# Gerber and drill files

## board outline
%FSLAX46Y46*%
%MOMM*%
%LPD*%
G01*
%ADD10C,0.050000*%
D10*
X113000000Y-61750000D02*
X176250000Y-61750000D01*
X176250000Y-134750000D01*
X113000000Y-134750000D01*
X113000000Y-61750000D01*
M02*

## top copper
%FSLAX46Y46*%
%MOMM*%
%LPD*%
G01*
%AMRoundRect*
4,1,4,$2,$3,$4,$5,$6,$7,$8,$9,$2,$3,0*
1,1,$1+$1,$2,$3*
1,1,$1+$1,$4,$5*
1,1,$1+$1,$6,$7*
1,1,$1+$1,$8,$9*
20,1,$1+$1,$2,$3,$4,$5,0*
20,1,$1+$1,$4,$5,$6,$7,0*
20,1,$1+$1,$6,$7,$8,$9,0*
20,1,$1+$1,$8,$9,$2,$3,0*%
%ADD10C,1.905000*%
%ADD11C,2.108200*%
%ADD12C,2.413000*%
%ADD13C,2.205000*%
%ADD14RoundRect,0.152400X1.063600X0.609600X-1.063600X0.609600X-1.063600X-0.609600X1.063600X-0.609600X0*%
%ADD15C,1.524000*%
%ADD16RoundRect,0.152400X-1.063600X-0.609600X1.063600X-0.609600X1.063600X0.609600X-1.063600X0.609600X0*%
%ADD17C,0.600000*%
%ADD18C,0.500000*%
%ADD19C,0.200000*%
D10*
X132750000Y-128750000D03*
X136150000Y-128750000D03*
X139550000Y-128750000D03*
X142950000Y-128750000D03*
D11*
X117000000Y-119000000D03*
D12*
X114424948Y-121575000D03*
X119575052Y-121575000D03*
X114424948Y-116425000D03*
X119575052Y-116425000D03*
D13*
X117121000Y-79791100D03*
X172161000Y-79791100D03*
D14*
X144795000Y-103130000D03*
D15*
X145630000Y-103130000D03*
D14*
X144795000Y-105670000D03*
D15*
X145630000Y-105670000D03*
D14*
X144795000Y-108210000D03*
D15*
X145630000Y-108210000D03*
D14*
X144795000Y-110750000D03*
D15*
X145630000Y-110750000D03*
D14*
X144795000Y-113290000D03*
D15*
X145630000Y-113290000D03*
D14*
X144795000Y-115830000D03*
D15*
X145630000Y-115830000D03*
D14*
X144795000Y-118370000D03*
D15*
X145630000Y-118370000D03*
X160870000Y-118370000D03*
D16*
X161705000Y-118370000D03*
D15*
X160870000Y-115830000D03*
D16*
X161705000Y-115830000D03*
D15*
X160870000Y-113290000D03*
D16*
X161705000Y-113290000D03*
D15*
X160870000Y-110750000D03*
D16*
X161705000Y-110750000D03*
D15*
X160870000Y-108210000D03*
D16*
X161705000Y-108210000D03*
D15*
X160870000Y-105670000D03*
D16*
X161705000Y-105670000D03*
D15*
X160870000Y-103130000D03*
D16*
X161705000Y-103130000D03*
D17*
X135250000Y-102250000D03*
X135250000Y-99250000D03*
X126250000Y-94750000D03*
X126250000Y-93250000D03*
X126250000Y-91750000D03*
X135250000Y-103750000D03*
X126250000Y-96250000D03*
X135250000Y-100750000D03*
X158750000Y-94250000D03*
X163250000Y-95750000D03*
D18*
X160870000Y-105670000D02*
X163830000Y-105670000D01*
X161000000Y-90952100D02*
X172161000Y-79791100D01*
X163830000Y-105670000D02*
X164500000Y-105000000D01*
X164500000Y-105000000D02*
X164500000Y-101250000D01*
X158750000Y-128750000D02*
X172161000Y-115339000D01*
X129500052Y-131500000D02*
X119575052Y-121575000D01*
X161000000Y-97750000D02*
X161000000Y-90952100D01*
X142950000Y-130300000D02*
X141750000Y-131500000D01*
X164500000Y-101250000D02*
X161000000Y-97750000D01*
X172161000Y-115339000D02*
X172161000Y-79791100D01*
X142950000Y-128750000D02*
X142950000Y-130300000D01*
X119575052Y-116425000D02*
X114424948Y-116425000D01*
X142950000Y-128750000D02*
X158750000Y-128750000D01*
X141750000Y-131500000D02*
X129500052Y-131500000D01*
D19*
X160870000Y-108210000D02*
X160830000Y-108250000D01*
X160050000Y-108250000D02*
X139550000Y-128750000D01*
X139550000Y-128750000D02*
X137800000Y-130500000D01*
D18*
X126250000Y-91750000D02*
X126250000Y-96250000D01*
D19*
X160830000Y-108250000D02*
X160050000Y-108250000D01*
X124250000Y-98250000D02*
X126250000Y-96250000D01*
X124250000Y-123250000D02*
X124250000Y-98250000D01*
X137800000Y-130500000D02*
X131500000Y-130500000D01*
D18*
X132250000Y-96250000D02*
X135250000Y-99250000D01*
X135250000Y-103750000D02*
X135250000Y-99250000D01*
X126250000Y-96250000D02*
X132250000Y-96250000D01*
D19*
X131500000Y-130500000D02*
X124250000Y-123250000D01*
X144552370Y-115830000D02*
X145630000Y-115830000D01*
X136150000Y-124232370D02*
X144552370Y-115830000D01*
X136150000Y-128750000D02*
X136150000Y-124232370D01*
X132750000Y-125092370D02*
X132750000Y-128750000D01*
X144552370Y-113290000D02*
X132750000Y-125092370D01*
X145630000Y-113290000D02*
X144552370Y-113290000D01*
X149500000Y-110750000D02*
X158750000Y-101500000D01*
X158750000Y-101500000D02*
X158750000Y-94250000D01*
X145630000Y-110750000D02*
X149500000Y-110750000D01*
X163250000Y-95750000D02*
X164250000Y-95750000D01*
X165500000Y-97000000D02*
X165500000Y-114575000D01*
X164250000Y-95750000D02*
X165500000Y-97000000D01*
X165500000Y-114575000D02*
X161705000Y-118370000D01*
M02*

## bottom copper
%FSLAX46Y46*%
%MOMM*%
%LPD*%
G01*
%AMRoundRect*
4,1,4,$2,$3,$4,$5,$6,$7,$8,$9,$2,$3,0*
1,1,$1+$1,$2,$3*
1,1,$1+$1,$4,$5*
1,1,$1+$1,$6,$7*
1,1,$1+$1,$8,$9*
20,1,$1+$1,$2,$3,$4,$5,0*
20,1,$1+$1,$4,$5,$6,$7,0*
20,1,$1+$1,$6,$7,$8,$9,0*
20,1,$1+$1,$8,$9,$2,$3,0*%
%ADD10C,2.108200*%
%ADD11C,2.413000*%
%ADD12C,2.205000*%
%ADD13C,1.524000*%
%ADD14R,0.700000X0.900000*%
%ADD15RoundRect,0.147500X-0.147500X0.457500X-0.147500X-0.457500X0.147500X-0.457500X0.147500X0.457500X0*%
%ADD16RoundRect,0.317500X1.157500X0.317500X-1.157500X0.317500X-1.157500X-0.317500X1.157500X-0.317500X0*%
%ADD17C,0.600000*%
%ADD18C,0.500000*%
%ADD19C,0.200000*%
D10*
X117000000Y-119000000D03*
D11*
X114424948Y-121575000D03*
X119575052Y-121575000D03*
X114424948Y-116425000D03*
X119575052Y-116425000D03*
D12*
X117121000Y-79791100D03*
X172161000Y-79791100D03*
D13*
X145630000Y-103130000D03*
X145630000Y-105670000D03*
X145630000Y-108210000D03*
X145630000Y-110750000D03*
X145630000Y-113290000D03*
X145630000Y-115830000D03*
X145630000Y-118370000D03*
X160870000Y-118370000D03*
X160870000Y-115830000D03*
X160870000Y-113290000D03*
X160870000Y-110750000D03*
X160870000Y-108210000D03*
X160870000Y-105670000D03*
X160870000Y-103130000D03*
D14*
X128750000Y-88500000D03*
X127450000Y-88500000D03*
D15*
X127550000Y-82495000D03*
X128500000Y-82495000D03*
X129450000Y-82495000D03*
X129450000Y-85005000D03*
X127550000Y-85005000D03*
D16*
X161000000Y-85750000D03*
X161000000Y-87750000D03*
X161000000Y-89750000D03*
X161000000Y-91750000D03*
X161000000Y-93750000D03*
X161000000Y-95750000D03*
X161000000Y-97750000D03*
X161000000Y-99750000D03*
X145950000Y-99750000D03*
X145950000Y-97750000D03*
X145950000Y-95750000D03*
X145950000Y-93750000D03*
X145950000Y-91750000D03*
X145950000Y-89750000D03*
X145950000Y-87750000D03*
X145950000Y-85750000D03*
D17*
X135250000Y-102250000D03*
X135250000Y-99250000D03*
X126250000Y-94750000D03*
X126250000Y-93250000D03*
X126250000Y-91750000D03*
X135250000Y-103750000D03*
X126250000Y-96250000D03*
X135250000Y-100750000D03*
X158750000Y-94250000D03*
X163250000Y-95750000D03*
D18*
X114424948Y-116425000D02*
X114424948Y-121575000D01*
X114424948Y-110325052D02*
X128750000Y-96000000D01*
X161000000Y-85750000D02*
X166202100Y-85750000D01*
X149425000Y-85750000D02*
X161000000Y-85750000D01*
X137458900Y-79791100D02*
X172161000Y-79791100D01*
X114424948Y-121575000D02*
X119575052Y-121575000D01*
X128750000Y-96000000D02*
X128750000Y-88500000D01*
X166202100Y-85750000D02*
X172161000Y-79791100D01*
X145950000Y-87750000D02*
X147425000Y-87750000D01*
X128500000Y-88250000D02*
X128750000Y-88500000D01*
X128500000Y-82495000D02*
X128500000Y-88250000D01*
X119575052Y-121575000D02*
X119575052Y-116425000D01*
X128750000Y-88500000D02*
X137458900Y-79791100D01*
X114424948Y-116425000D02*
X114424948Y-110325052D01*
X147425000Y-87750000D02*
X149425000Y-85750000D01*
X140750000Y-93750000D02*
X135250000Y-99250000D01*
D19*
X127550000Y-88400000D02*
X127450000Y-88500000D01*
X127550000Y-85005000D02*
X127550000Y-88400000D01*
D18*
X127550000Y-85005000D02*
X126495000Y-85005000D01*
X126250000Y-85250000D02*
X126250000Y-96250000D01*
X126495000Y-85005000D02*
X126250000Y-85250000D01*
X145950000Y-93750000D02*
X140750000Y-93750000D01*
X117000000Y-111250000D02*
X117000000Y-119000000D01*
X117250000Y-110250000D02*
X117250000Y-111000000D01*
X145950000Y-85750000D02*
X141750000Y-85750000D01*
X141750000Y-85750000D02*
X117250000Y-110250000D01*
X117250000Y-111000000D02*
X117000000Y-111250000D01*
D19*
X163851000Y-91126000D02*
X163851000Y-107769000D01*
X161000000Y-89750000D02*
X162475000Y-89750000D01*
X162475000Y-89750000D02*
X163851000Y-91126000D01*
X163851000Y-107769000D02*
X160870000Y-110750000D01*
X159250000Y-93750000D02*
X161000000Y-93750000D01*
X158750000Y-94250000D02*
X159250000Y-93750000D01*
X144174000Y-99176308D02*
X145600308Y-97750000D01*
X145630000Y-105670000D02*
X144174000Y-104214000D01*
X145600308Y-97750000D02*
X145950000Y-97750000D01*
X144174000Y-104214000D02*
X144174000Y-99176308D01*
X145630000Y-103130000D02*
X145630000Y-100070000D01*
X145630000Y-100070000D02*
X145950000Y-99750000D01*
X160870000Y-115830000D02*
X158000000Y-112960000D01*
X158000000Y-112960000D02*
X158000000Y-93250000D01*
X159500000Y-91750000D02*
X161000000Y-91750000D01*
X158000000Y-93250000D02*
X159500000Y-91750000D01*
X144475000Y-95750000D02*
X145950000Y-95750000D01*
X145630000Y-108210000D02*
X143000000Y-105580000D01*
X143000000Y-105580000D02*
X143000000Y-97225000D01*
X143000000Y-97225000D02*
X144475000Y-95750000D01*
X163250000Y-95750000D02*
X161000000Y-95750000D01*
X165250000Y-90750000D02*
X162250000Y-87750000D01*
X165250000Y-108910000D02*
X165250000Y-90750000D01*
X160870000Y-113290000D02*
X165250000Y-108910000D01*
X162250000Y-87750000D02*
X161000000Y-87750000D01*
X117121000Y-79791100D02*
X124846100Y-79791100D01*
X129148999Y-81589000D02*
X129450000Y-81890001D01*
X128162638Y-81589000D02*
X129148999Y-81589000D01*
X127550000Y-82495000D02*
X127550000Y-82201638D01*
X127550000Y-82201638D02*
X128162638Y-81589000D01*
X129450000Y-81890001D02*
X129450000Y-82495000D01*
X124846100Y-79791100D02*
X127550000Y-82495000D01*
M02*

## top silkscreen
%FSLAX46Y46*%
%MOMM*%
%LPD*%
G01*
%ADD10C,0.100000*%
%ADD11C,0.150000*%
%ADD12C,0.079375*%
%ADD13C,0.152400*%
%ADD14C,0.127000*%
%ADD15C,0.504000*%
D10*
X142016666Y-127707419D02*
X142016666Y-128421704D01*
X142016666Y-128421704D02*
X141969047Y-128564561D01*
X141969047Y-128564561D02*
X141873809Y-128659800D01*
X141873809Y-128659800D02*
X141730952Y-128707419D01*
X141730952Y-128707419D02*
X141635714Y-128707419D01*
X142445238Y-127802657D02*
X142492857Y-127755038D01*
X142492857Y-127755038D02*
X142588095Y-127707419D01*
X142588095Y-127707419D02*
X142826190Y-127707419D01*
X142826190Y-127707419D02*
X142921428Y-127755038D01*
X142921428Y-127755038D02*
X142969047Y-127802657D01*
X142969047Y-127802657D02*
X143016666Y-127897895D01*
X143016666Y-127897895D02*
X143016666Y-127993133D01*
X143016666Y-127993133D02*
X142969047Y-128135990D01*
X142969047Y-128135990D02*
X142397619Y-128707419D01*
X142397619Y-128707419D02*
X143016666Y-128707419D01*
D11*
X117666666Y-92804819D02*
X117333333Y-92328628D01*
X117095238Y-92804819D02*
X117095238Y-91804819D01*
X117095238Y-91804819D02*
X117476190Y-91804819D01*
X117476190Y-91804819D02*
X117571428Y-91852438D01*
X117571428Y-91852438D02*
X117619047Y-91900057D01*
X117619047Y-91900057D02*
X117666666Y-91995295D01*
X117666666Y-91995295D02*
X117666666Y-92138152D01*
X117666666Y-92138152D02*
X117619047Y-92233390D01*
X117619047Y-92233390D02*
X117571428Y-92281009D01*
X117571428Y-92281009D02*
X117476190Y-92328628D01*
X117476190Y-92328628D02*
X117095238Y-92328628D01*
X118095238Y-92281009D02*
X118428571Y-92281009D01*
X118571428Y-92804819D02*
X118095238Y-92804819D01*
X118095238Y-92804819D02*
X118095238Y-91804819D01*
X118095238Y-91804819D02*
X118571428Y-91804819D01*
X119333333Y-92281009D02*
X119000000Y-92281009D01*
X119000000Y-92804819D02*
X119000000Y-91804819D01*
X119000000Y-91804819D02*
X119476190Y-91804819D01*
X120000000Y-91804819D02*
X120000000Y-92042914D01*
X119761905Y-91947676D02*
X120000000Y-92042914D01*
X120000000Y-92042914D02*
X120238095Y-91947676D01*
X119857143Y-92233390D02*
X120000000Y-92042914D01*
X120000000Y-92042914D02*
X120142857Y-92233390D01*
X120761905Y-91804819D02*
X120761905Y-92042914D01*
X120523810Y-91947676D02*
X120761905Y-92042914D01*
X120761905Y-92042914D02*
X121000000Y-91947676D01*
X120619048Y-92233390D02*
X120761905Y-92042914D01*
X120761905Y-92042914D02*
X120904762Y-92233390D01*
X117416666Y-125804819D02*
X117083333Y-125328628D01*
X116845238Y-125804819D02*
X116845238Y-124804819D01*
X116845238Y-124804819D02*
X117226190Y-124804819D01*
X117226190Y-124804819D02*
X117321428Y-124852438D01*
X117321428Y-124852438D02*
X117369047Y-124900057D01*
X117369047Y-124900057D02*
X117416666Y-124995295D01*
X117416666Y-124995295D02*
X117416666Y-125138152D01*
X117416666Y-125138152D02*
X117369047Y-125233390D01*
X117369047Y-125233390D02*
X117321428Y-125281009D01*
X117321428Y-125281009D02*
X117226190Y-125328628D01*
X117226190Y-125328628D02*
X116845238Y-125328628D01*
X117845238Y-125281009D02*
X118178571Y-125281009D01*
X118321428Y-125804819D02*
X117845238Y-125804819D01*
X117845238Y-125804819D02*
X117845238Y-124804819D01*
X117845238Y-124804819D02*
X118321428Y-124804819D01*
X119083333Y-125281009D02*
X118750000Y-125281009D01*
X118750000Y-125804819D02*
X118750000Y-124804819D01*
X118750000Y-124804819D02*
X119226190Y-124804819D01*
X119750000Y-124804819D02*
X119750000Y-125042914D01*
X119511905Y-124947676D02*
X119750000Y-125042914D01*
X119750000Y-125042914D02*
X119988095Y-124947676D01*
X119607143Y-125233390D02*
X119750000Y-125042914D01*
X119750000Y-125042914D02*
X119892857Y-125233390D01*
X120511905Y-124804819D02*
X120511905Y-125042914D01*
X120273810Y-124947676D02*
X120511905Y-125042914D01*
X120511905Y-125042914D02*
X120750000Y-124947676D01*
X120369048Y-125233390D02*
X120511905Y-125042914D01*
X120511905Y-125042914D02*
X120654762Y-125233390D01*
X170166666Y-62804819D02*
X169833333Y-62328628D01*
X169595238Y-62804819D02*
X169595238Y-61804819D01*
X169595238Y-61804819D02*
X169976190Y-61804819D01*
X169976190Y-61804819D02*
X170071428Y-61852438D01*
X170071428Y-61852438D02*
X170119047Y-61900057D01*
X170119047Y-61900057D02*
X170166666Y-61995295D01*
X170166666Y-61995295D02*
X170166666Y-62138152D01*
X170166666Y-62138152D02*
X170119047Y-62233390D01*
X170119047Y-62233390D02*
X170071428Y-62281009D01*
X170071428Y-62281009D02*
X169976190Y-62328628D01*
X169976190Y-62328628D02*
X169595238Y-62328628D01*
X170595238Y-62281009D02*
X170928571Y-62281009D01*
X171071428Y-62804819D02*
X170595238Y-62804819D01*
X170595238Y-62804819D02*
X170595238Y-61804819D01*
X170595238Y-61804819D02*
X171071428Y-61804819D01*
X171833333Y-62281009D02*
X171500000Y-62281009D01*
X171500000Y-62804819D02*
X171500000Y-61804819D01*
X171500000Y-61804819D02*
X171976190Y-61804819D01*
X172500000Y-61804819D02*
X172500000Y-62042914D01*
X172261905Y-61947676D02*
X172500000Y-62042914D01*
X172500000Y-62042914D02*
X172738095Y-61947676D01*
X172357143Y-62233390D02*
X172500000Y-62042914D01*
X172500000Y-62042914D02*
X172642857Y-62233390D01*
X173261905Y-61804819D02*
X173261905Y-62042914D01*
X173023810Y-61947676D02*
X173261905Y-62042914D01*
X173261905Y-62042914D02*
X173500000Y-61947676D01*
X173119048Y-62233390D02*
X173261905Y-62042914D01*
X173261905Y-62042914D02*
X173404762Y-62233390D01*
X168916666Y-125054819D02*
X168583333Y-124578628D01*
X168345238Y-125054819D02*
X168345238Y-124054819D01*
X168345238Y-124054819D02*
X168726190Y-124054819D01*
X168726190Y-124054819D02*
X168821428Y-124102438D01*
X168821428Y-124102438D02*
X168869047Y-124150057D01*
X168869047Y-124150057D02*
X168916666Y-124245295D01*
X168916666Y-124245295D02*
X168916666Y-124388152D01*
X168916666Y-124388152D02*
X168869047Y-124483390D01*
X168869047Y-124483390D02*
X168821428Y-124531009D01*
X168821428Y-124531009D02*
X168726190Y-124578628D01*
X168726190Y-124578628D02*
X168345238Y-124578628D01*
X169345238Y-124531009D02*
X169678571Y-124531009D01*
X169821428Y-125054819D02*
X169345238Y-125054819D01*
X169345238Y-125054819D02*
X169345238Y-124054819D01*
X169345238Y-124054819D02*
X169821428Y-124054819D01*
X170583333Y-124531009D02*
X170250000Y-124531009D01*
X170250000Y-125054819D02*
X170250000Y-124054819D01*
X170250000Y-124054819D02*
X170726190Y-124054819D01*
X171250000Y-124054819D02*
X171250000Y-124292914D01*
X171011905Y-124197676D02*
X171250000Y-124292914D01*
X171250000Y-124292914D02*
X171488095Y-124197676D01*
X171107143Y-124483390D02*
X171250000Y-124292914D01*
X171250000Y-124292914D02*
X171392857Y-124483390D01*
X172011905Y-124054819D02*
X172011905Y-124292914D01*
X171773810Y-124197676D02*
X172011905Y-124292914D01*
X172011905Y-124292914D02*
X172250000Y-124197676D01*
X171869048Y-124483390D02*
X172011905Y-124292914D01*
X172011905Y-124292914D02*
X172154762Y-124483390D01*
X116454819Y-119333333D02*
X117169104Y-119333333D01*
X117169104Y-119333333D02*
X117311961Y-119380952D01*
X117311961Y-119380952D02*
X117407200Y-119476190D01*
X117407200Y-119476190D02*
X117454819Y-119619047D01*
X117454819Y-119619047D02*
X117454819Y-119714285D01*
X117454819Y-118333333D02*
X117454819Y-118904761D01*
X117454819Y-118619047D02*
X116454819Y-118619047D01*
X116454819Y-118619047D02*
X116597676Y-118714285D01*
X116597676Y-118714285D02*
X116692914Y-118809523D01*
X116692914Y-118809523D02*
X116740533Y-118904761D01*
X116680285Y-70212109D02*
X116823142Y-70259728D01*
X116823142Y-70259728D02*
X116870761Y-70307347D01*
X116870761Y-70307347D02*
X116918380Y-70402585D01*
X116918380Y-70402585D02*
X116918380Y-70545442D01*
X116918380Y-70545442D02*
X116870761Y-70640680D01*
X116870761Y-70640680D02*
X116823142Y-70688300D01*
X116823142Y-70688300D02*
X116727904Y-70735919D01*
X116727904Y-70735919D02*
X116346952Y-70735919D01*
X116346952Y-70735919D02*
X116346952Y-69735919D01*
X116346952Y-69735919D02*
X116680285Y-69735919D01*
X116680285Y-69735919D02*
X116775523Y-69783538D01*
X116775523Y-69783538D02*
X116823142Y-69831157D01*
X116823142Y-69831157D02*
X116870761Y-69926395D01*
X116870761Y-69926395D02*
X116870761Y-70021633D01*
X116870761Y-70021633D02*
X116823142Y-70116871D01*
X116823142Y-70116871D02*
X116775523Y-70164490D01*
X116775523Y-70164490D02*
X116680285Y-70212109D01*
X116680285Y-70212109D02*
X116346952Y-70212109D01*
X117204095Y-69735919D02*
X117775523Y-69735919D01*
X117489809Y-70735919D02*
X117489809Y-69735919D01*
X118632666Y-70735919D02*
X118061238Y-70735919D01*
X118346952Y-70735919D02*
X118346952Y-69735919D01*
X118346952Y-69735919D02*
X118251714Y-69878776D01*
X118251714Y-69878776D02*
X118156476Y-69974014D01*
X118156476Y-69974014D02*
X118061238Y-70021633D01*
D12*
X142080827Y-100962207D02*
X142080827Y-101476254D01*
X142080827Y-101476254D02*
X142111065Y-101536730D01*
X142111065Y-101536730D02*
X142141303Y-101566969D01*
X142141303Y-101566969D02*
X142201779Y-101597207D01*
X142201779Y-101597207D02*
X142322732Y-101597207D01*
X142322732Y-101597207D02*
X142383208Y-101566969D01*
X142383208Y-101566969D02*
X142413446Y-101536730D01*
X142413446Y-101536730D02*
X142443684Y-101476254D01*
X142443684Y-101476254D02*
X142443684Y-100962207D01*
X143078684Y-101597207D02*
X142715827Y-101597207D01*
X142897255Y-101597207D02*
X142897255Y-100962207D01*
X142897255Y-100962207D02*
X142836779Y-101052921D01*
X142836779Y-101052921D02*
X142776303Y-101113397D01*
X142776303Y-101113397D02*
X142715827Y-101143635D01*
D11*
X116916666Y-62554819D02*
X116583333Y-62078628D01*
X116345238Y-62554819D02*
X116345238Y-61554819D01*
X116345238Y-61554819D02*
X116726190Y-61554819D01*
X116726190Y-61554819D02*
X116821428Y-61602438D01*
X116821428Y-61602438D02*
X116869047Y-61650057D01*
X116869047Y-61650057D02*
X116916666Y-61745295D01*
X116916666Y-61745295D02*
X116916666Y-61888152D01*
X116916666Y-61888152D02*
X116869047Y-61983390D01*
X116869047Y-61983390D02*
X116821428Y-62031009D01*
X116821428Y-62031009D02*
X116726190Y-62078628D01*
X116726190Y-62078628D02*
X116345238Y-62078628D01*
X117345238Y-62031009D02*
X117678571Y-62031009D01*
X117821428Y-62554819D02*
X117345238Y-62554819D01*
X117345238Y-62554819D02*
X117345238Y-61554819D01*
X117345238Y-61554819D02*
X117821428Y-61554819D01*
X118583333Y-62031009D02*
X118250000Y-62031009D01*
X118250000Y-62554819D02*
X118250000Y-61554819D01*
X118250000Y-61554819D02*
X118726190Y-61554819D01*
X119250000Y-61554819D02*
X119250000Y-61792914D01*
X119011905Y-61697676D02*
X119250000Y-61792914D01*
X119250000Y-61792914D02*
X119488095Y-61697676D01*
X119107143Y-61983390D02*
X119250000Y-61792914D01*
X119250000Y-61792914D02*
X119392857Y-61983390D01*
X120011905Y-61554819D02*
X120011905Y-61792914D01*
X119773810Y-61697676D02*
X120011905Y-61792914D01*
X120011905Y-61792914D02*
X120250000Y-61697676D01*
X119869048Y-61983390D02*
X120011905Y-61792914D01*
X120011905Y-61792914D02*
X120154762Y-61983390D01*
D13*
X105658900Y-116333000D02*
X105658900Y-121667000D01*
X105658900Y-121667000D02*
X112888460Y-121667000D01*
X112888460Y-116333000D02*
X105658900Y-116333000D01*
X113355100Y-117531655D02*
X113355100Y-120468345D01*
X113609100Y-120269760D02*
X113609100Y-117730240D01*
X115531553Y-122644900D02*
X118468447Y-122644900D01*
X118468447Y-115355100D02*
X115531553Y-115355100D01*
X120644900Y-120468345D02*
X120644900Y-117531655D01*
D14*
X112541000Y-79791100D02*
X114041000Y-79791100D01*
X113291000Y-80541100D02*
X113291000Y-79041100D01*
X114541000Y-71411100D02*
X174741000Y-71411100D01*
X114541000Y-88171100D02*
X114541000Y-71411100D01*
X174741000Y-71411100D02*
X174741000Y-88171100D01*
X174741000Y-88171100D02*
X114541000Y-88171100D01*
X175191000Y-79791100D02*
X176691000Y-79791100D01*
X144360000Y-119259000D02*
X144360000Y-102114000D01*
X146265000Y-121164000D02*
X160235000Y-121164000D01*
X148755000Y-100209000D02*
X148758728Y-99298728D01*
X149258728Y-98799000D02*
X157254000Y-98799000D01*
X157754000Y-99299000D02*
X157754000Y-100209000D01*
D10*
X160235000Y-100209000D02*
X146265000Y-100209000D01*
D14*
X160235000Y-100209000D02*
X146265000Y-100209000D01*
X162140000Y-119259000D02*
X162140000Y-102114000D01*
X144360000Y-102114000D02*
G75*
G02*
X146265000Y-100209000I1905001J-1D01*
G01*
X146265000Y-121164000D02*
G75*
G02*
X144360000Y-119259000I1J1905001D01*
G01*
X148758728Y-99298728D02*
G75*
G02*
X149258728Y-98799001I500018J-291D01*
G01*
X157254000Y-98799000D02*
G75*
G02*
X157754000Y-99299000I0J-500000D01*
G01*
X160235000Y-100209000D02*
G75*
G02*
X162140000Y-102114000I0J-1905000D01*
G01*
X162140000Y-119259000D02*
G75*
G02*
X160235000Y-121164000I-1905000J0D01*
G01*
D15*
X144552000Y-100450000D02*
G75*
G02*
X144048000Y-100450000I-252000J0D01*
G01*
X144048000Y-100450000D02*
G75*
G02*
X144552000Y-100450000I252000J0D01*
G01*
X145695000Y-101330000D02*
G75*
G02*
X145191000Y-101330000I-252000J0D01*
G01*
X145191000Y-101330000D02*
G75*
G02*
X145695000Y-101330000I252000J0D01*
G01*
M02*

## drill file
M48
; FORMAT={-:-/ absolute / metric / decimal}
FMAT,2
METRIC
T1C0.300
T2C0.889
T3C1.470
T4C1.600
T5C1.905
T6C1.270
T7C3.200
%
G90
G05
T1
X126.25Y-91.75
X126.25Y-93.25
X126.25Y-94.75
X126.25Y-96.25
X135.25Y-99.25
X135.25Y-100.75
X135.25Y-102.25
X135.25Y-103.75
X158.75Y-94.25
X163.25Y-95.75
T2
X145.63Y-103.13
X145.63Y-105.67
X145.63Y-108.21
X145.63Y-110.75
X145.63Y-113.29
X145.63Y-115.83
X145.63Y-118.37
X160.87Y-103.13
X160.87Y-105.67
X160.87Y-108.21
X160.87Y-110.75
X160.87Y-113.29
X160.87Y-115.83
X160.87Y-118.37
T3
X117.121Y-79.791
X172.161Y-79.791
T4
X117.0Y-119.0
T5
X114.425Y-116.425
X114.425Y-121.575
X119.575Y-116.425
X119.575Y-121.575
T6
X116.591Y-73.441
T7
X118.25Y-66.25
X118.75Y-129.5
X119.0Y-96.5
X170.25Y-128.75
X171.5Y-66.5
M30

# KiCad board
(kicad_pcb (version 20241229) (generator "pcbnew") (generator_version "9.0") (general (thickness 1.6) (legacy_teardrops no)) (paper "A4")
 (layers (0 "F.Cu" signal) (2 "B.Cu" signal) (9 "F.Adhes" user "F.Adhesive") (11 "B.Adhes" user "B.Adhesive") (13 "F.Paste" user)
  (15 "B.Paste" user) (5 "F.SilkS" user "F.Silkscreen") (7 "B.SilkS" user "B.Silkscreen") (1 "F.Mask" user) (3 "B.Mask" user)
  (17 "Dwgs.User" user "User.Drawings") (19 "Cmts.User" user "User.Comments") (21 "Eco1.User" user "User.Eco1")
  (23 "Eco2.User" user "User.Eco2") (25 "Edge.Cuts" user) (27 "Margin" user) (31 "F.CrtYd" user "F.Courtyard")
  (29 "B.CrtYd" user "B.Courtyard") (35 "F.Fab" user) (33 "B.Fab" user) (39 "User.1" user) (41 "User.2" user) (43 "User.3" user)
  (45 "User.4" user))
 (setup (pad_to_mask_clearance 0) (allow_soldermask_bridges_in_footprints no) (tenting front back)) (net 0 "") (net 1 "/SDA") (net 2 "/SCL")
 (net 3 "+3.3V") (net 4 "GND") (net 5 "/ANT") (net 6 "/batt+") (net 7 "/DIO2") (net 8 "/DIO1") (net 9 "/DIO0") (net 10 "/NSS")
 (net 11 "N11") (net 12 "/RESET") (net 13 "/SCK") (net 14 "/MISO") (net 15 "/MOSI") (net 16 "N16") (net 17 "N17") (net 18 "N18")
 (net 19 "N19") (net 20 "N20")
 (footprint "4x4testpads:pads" (layer "F.Cu") (at 142.35 128.75)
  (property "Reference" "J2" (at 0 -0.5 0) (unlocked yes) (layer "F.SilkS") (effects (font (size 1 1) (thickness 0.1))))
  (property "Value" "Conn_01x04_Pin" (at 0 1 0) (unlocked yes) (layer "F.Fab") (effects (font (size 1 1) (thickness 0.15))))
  (pad "1" smd circle (at -9.6 0) (size 1.905 1.905) (layers "F.Cu" "F.Mask" "F.Paste") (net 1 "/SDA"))
  (pad "2" smd circle (at -6.2 0) (size 1.905 1.905) (layers "F.Cu" "F.Mask" "F.Paste") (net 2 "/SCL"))
  (pad "3" smd circle (at -2.8 0) (size 1.905 1.905) (layers "F.Cu" "F.Mask" "F.Paste") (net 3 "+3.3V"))
  (pad "4" smd circle (at 0.6 0) (size 1.905 1.905) (layers "F.Cu" "F.Mask" "F.Paste") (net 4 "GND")))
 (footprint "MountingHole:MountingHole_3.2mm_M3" (layer "F.Cu") (at 119 96.5)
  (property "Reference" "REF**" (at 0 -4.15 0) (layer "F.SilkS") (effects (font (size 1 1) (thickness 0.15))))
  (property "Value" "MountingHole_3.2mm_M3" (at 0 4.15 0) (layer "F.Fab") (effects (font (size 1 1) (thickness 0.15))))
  (pad "" np_thru_hole circle (at 0 0) (size 3.2 3.2) (drill 3.2) (layers "*.Cu" "*.Mask")))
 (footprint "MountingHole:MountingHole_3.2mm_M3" (layer "F.Cu") (at 118.75 129.5)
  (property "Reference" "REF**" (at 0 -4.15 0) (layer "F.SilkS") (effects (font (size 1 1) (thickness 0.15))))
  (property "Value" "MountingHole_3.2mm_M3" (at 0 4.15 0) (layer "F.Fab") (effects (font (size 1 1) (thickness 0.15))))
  (pad "" np_thru_hole circle (at 0 0) (size 3.2 3.2) (drill 3.2) (layers "*.Cu" "*.Mask")))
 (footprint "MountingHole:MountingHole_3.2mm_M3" (layer "F.Cu") (at 171.5 66.5)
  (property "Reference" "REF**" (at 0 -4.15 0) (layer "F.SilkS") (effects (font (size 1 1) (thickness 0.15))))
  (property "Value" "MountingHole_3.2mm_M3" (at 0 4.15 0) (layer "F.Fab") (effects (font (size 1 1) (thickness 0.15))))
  (pad "" np_thru_hole circle (at 0 0) (size 3.2 3.2) (drill 3.2) (layers "*.Cu" "*.Mask")))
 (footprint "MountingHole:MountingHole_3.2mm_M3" (layer "F.Cu") (at 170.25 128.75)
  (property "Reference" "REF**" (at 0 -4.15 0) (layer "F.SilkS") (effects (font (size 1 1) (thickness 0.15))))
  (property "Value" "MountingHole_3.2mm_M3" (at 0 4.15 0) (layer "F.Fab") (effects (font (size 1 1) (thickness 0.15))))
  (pad "" np_thru_hole circle (at 0 0) (size 3.2 3.2) (drill 3.2) (layers "*.Cu" "*.Mask")))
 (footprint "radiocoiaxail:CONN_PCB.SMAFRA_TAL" (layer "F.Cu") (at 117 119 90)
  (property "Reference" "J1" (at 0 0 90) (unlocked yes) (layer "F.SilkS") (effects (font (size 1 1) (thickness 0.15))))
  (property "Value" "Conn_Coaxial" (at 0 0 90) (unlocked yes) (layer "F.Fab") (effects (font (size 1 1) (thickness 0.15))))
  (fp_line (start 2.667 -11.3411) (end -2.667 -11.3411) (stroke (width 0.1524) (type solid)) (layer "F.SilkS"))
  (fp_line (start -2.667 -11.3411) (end -2.667 -4.11154) (stroke (width 0.1524) (type solid)) (layer "F.SilkS"))
  (fp_line (start 2.667 -4.11154) (end 2.667 -11.3411) (stroke (width 0.1524) (type solid)) (layer "F.SilkS"))
  (fp_line (start 1.468345 -3.6449) (end -1.468345 -3.6449) (stroke (width 0.1524) (type solid)) (layer "F.SilkS"))
  (fp_line (start -1.26976 -3.3909) (end 1.26976 -3.3909) (stroke (width 0.1524) (type solid)) (layer "F.SilkS"))
  (fp_line (start -3.6449 -1.468447) (end -3.6449 1.468447) (stroke (width 0.1524) (type solid)) (layer "F.SilkS"))
  (fp_line (start 3.6449 1.468447) (end 3.6449 -1.468447) (stroke (width 0.1524) (type solid)) (layer "F.SilkS"))
  (fp_line (start -1.468345 3.6449) (end 1.468345 3.6449) (stroke (width 0.1524) (type solid)) (layer "F.SilkS"))
  (pad "1" thru_hole circle (at 0 0 90) (size 2.1082 2.1082) (drill 1.6002) (layers "*.Cu" "*.Mask") (remove_unused_layers no)
   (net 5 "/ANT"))
  (pad "2" thru_hole circle (at -2.575 -2.575052 90) (size 2.413 2.413) (drill 1.905) (layers "*.Cu" "*.Mask") (remove_unused_layers no)
   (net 4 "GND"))
  (pad "2" thru_hole circle (at -2.575 2.575052 90) (size 2.413 2.413) (drill 1.905) (layers "*.Cu" "*.Mask") (remove_unused_layers no)
   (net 4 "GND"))
  (pad "2" thru_hole circle (at 2.575 -2.575052 90) (size 2.413 2.413) (drill 1.905) (layers "*.Cu" "*.Mask") (remove_unused_layers no)
   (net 4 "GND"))
  (pad "2" thru_hole circle (at 2.575 2.575052 90) (size 2.413 2.413) (drill 1.905) (layers "*.Cu" "*.Mask") (remove_unused_layers no)
   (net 4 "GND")))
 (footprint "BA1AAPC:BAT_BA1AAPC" (layer "F.Cu") (at 144.641 79.7911)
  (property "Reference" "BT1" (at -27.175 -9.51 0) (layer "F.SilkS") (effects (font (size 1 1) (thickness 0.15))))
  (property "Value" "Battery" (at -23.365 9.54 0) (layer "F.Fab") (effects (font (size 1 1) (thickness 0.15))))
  (fp_line (start -32.1 0) (end -30.6 0) (stroke (width 0.127) (type solid)) (layer "F.SilkS"))
  (fp_line (start -31.35 0.75) (end -31.35 -0.75) (stroke (width 0.127) (type solid)) (layer "F.SilkS"))
  (fp_line (start -30.1 -8.38) (end 30.1 -8.38) (stroke (width 0.127) (type solid)) (layer "F.SilkS"))
  (fp_line (start -30.1 8.38) (end -30.1 -8.38) (stroke (width 0.127) (type solid)) (layer "F.SilkS"))
  (fp_line (start 30.1 -8.38) (end 30.1 8.38) (stroke (width 0.127) (type solid)) (layer "F.SilkS"))
  (fp_line (start 30.1 8.38) (end -30.1 8.38) (stroke (width 0.127) (type solid)) (layer "F.SilkS"))
  (fp_line (start 30.55 0) (end 32.05 0) (stroke (width 0.127) (type solid)) (layer "F.SilkS"))
  (pad "" np_thru_hole circle (at -28.05 -6.35) (size 1.27 1.27) (drill 1.27) (layers "*.Cu" "*.Mask"))
  (pad "1" thru_hole circle (at -27.52 0) (size 2.205 2.205) (drill 1.47) (layers "*.Cu" "*.Mask") (remove_unused_layers no)
   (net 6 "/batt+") (solder_mask_margin 0.102))
  (pad "2" thru_hole circle (at 27.52 0) (size 2.205 2.205) (drill 1.47) (layers "*.Cu" "*.Mask") (remove_unused_layers no) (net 4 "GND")
   (solder_mask_margin 0.102)))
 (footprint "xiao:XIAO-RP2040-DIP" (layer "F.Cu") (at 153.25 110.75)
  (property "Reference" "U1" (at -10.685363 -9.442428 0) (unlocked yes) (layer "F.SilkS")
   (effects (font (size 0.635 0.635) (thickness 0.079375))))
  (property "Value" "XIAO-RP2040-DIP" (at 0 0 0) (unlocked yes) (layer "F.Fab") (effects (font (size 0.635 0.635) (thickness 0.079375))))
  (fp_line (start -8.89 8.509) (end -8.89 -8.636) (stroke (width 0.127) (type solid)) (layer "F.SilkS"))
  (fp_line (start -6.985 10.414) (end 6.985 10.414) (stroke (width 0.127) (type solid)) (layer "F.SilkS"))
  (fp_line (start -4.495 -10.541) (end -4.491272 -11.451272) (stroke (width 0.127) (type solid)) (layer "F.SilkS"))
  (fp_line (start -3.991272 -11.951) (end 4.004 -11.951) (stroke (width 0.127) (type solid)) (layer "F.SilkS"))
  (fp_line (start 4.504 -11.451) (end 4.504 -10.541) (stroke (width 0.127) (type solid)) (layer "F.SilkS"))
  (fp_line (start 6.985 -10.541) (end -6.985 -10.541) (stroke (width 0.1) (type solid)) (layer "F.SilkS"))
  (fp_line (start 6.985 -10.541) (end -6.985 -10.541) (stroke (width 0.127) (type solid)) (layer "F.SilkS"))
  (fp_line (start 8.89 8.509) (end 8.89 -8.636) (stroke (width 0.127) (type solid)) (layer "F.SilkS"))
  (fp_arc (start -8.89 -8.636) (mid -8.332038 -9.983038) (end -6.985 -10.541) (stroke (width 0.127) (type solid)) (layer "F.SilkS"))
  (fp_arc (start -6.985 10.414) (mid -8.332038 9.856038) (end -8.89 8.509) (stroke (width 0.127) (type solid)) (layer "F.SilkS"))
  (fp_arc (start -4.491272 -11.451272) (mid -4.344728 -11.80464) (end -3.991272 -11.951) (stroke (width 0.127) (type default))
   (layer "F.SilkS"))
  (fp_arc (start 4.004 -11.951) (mid 4.357553 -11.804553) (end 4.504 -11.451) (stroke (width 0.127) (type default)) (layer "F.SilkS"))
  (fp_arc (start 6.985 -10.541) (mid 8.332038 -9.983038) (end 8.89 -8.636) (stroke (width 0.127) (type solid)) (layer "F.SilkS"))
  (fp_arc (start 8.89 8.509) (mid 8.332038 9.856038) (end 6.985 10.414) (stroke (width 0.127) (type solid)) (layer "F.SilkS"))
  (fp_circle (center -8.95 -10.3) (end -8.95 -10.554) (stroke (width 0.5) (type solid)) (fill yes) (layer "F.SilkS"))
  (fp_circle (center -7.807 -9.42) (end -7.807 -9.674) (stroke (width 0.5) (type solid)) (fill yes) (layer "F.SilkS"))
  (pad "1" smd roundrect (at -8.455 -7.62 180) (size 2.432 1.524) (layers "F.Cu" "F.Mask") (roundrect_rratio 0.1) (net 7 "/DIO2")
   (thermal_bridge_angle 45))
  (pad "1" thru_hole circle (at -7.62 -7.62 180) (size 1.524 1.524) (drill 0.889) (layers "*.Cu" "*.Mask") (remove_unused_layers no)
   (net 7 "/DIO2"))
  (pad "2" smd roundrect (at -8.455 -5.08 180) (size 2.432 1.524) (layers "F.Cu" "F.Mask") (roundrect_rratio 0.1) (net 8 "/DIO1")
   (thermal_bridge_angle 45))
  (pad "2" thru_hole circle (at -7.62 -5.08 180) (size 1.524 1.524) (drill 0.889) (layers "*.Cu" "*.Mask") (remove_unused_layers no)
   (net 8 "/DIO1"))
  (pad "3" smd roundrect (at -8.455 -2.54 180) (size 2.432 1.524) (layers "F.Cu" "F.Mask") (roundrect_rratio 0.1) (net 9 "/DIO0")
   (thermal_bridge_angle 45))
  (pad "3" thru_hole circle (at -7.62 -2.54 180) (size 1.524 1.524) (drill 0.889) (layers "*.Cu" "*.Mask") (remove_unused_layers no)
   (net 9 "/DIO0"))
  (pad "4" smd roundrect (at -8.455 0 180) (size 2.432 1.524) (layers "F.Cu" "F.Mask") (roundrect_rratio 0.1) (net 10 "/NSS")
   (thermal_bridge_angle 45))
  (pad "4" thru_hole circle (at -7.62 0 180) (size 1.524 1.524) (drill 0.889) (layers "*.Cu" "*.Mask") (remove_unused_layers no)
   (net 10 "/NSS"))
  (pad "5" smd roundrect (at -8.455 2.54 180) (size 2.432 1.524) (layers "F.Cu" "F.Mask") (roundrect_rratio 0.1) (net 1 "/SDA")
   (thermal_bridge_angle 45))
  (pad "5" thru_hole circle (at -7.62 2.54 180) (size 1.524 1.524) (drill 0.889) (layers "*.Cu" "*.Mask") (remove_unused_layers no)
   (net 1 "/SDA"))
  (pad "6" smd roundrect (at -8.455 5.08 180) (size 2.432 1.524) (layers "F.Cu" "F.Mask") (roundrect_rratio 0.1) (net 2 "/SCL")
   (thermal_bridge_angle 45))
  (pad "6" thru_hole circle (at -7.62 5.08 180) (size 1.524 1.524) (drill 0.889) (layers "*.Cu" "*.Mask") (remove_unused_layers no)
   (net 2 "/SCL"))
  (pad "7" smd roundrect (at -8.455 7.62 180) (size 2.432 1.524) (layers "F.Cu" "F.Mask") (roundrect_rratio 0.1) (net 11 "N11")
   (thermal_bridge_angle 45))
  (pad "7" thru_hole circle (at -7.62 7.62 180) (size 1.524 1.524) (drill 0.889) (layers "*.Cu" "*.Mask") (remove_unused_layers no)
   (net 11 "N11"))
  (pad "8" thru_hole circle (at 7.62 7.62) (size 1.524 1.524) (drill 0.889) (layers "*.Cu" "*.Mask") (remove_unused_layers no)
   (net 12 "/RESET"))
  (pad "8" smd roundrect (at 8.455 7.62) (size 2.432 1.524) (layers "F.Cu" "F.Mask") (roundrect_rratio 0.1) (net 12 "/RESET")
   (thermal_bridge_angle 45))
  (pad "9" thru_hole circle (at 7.62 5.08) (size 1.524 1.524) (drill 0.889) (layers "*.Cu" "*.Mask") (remove_unused_layers no)
   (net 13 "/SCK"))
  (pad "9" smd roundrect (at 8.455 5.08) (size 2.432 1.524) (layers "F.Cu" "F.Mask") (roundrect_rratio 0.1) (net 13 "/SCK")
   (thermal_bridge_angle 45))
  (pad "10" thru_hole circle (at 7.62 2.54) (size 1.524 1.524) (drill 0.889) (layers "*.Cu" "*.Mask") (remove_unused_layers no)
   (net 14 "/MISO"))
  (pad "10" smd roundrect (at 8.455 2.54) (size 2.432 1.524) (layers "F.Cu" "F.Mask") (roundrect_rratio 0.1) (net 14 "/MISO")
   (thermal_bridge_angle 45))
  (pad "11" thru_hole circle (at 7.62 0) (size 1.524 1.524) (drill 0.889) (layers "*.Cu" "*.Mask") (remove_unused_layers no)
   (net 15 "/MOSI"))
  (pad "11" smd roundrect (at 8.455 0) (size 2.432 1.524) (layers "F.Cu" "F.Mask") (roundrect_rratio 0.1) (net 15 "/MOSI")
   (thermal_bridge_angle 45))
  (pad "12" thru_hole circle (at 7.62 -2.54) (size 1.524 1.524) (drill 0.889) (layers "*.Cu" "*.Mask") (remove_unused_layers no)
   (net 3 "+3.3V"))
  (pad "12" smd roundrect (at 8.455 -2.54) (size 2.432 1.524) (layers "F.Cu" "F.Mask") (roundrect_rratio 0.1) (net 3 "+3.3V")
   (thermal_bridge_angle 45))
  (pad "13" thru_hole circle (at 7.62 -5.08) (size 1.524 1.524) (drill 0.889) (layers "*.Cu" "*.Mask") (remove_unused_layers no)
   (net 4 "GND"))
  (pad "13" smd roundrect (at 8.455 -5.08) (size 2.432 1.524) (layers "F.Cu" "F.Mask") (roundrect_rratio 0.1) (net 4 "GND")
   (thermal_bridge_angle 45))
  (pad "14" thru_hole circle (at 7.62 -7.62) (size 1.524 1.524) (drill 0.889) (layers "*.Cu" "*.Mask") (remove_unused_layers no)
   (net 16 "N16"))
  (pad "14" smd roundrect (at 8.455 -7.62) (size 2.432 1.524) (layers "F.Cu" "F.Mask") (roundrect_rratio 0.1) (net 16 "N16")
   (thermal_bridge_angle 45)))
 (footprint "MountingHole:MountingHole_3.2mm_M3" (layer "F.Cu") (at 118.25 66.25)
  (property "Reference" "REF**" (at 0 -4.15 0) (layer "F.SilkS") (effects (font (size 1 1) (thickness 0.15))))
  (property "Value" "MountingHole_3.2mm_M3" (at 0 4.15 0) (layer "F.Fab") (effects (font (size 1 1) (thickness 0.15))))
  (pad "" np_thru_hole circle (at 0 0) (size 3.2 3.2) (drill 3.2) (layers "*.Cu" "*.Mask")))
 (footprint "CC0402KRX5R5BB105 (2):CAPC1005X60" (layer "B.Cu") (at 128.1 88.5 180)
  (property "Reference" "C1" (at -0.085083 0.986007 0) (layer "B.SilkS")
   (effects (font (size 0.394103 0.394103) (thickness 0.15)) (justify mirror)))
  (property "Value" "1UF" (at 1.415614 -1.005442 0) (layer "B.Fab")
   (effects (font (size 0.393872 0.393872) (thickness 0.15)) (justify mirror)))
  (pad "1" smd rect (at -0.65 0 180) (size 0.7 0.9) (layers "B.Cu" "B.Mask" "B.Paste") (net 4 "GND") (solder_mask_margin 0.102))
  (pad "2" smd rect (at 0.65 0 180) (size 0.7 0.9) (layers "B.Cu" "B.Mask" "B.Paste") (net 3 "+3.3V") (solder_mask_margin 0.102)))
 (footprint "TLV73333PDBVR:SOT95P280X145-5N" (layer "B.Cu") (at 128.5 83.75 -90)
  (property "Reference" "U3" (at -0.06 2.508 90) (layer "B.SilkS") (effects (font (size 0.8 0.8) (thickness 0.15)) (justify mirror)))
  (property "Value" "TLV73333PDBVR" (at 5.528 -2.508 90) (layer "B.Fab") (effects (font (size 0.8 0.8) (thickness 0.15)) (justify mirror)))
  (pad "1" smd roundrect (at -1.255 0.95 270) (size 1.21 0.59) (layers "B.Cu" "B.Mask" "B.Paste") (roundrect_rratio 0.25) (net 6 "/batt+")
   (solder_mask_margin 0.102))
  (pad "2" smd roundrect (at -1.255 0 270) (size 1.21 0.59) (layers "B.Cu" "B.Mask" "B.Paste") (roundrect_rratio 0.25) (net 4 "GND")
   (solder_mask_margin 0.102))
  (pad "3" smd roundrect (at -1.255 -0.95 270) (size 1.21 0.59) (layers "B.Cu" "B.Mask" "B.Paste") (roundrect_rratio 0.25) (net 6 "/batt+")
   (solder_mask_margin 0.102))
  (pad "4" smd roundrect (at 1.255 -0.95 270) (size 1.21 0.59) (layers "B.Cu" "B.Mask" "B.Paste") (roundrect_rratio 0.25) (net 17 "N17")
   (solder_mask_margin 0.102))
  (pad "5" smd roundrect (at 1.255 0.95 270) (size 1.21 0.59) (layers "B.Cu" "B.Mask" "B.Paste") (roundrect_rratio 0.25) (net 3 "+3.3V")
   (solder_mask_margin 0.102)))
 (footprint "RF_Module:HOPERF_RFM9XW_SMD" (layer "B.Cu") (at 153.475 92.75 180)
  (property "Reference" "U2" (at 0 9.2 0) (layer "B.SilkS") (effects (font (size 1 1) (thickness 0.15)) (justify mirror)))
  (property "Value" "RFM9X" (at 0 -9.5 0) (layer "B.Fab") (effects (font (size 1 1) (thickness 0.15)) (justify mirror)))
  (pad "1" smd roundrect (at -7.525 7 180) (size 2.95 1.27) (layers "B.Cu" "B.Mask" "B.Paste") (roundrect_rratio 0.25) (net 4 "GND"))
  (pad "2" smd roundrect (at -7.525 5 180) (size 2.95 1.27) (layers "B.Cu" "B.Mask" "B.Paste") (roundrect_rratio 0.25) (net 14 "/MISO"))
  (pad "3" smd roundrect (at -7.525 3 180) (size 2.95 1.27) (layers "B.Cu" "B.Mask" "B.Paste") (roundrect_rratio 0.25) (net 15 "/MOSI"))
  (pad "4" smd roundrect (at -7.525 1 180) (size 2.95 1.27) (layers "B.Cu" "B.Mask" "B.Paste") (roundrect_rratio 0.25) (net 13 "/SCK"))
  (pad "5" smd roundrect (at -7.525 -1 180) (size 2.95 1.27) (layers "B.Cu" "B.Mask" "B.Paste") (roundrect_rratio 0.25) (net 10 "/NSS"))
  (pad "6" smd roundrect (at -7.525 -3 180) (size 2.95 1.27) (layers "B.Cu" "B.Mask" "B.Paste") (roundrect_rratio 0.25) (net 12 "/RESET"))
  (pad "7" smd roundrect (at -7.525 -5 180) (size 2.95 1.27) (layers "B.Cu" "B.Mask" "B.Paste") (roundrect_rratio 0.25) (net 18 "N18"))
  (pad "8" smd roundrect (at -7.525 -7 180) (size 2.95 1.27) (layers "B.Cu" "B.Mask" "B.Paste") (roundrect_rratio 0.25) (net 4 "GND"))
  (pad "9" smd roundrect (at 7.525 -7 180) (size 2.95 1.27) (layers "B.Cu" "B.Mask" "B.Paste") (roundrect_rratio 0.25) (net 7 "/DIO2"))
  (pad "10" smd roundrect (at 7.525 -5 180) (size 2.95 1.27) (layers "B.Cu" "B.Mask" "B.Paste") (roundrect_rratio 0.25) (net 8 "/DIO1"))
  (pad "11" smd roundrect (at 7.525 -3 180) (size 2.95 1.27) (layers "B.Cu" "B.Mask" "B.Paste") (roundrect_rratio 0.25) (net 9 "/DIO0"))
  (pad "12" smd roundrect (at 7.525 -1 180) (size 2.95 1.27) (layers "B.Cu" "B.Mask" "B.Paste") (roundrect_rratio 0.25) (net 3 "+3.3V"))
  (pad "13" smd roundrect (at 7.525 1 180) (size 2.95 1.27) (layers "B.Cu" "B.Mask" "B.Paste") (roundrect_rratio 0.25) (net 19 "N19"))
  (pad "14" smd roundrect (at 7.525 3 180) (size 2.95 1.27) (layers "B.Cu" "B.Mask" "B.Paste") (roundrect_rratio 0.25) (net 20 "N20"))
  (pad "15" smd roundrect (at 7.525 5 180) (size 2.95 1.27) (layers "B.Cu" "B.Mask" "B.Paste") (roundrect_rratio 0.25) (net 4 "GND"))
  (pad "16" smd roundrect (at 7.525 7 180) (size 2.95 1.27) (layers "B.Cu" "B.Mask" "B.Paste") (roundrect_rratio 0.25) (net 5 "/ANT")))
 (gr_rect (start 113 61.75) (end 176.25 134.75) (stroke (width 0.05) (type default)) (fill no) (layer "Edge.Cuts"))
 (segment (start 160.87 105.67) (end 163.83 105.67) (width 0.5) (layer "F.Cu") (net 4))
 (segment (start 161 90.9521) (end 172.161 79.7911) (width 0.5) (layer "F.Cu") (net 4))
 (segment (start 163.83 105.67) (end 164.5 105) (width 0.5) (layer "F.Cu") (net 4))
 (segment (start 164.5 105) (end 164.5 101.25) (width 0.5) (layer "F.Cu") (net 4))
 (segment (start 158.75 128.75) (end 172.161 115.339) (width 0.5) (layer "F.Cu") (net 4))
 (segment (start 129.500052 131.5) (end 119.575052 121.575) (width 0.5) (layer "F.Cu") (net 4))
 (segment (start 161 97.75) (end 161 90.9521) (width 0.5) (layer "F.Cu") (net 4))
 (segment (start 142.95 130.3) (end 141.75 131.5) (width 0.5) (layer "F.Cu") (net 4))
 (segment (start 164.5 101.25) (end 161 97.75) (width 0.5) (layer "F.Cu") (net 4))
 (segment (start 172.161 115.339) (end 172.161 79.7911) (width 0.5) (layer "F.Cu") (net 4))
 (segment (start 142.95 128.75) (end 142.95 130.3) (width 0.5) (layer "F.Cu") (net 4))
 (segment (start 119.575052 116.425) (end 114.424948 116.425) (width 0.5) (layer "F.Cu") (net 4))
 (segment (start 142.95 128.75) (end 158.75 128.75) (width 0.5) (layer "F.Cu") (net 4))
 (segment (start 141.75 131.5) (end 129.500052 131.5) (width 0.5) (layer "F.Cu") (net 4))
 (segment (start 114.424948 116.425) (end 114.424948 121.575) (width 0.5) (layer "B.Cu") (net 4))
 (segment (start 114.424948 110.325052) (end 128.75 96) (width 0.5) (layer "B.Cu") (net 4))
 (segment (start 161 85.75) (end 166.2021 85.75) (width 0.5) (layer "B.Cu") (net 4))
 (segment (start 149.425 85.75) (end 161 85.75) (width 0.5) (layer "B.Cu") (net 4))
 (segment (start 137.4589 79.7911) (end 172.161 79.7911) (width 0.5) (layer "B.Cu") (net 4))
 (segment (start 114.424948 121.575) (end 119.575052 121.575) (width 0.5) (layer "B.Cu") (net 4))
 (segment (start 128.75 96) (end 128.75 88.5) (width 0.5) (layer "B.Cu") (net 4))
 (segment (start 166.2021 85.75) (end 172.161 79.7911) (width 0.5) (layer "B.Cu") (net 4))
 (segment (start 145.95 87.75) (end 147.425 87.75) (width 0.5) (layer "B.Cu") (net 4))
 (segment (start 128.5 88.25) (end 128.75 88.5) (width 0.5) (layer "B.Cu") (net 4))
 (segment (start 128.5 82.495) (end 128.5 88.25) (width 0.5) (layer "B.Cu") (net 4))
 (segment (start 119.575052 121.575) (end 119.575052 116.425) (width 0.5) (layer "B.Cu") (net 4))
 (segment (start 128.75 88.5) (end 137.4589 79.7911) (width 0.5) (layer "B.Cu") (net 4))
 (segment (start 114.424948 116.425) (end 114.424948 110.325052) (width 0.5) (layer "B.Cu") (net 4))
 (segment (start 147.425 87.75) (end 149.425 85.75) (width 0.5) (layer "B.Cu") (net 4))
 (segment (start 160.87 108.21) (end 160.83 108.25) (width 0.2) (layer "F.Cu") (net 3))
 (segment (start 160.05 108.25) (end 139.55 128.75) (width 0.2) (layer "F.Cu") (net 3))
 (segment (start 139.55 128.75) (end 137.8 130.5) (width 0.2) (layer "F.Cu") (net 3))
 (segment (start 126.25 91.75) (end 126.25 96.25) (width 0.5) (layer "F.Cu") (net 3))
 (segment (start 160.83 108.25) (end 160.05 108.25) (width 0.2) (layer "F.Cu") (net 3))
 (segment (start 124.25 98.25) (end 126.25 96.25) (width 0.2) (layer "F.Cu") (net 3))
 (segment (start 124.25 123.25) (end 124.25 98.25) (width 0.2) (layer "F.Cu") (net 3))
 (segment (start 137.8 130.5) (end 131.5 130.5) (width 0.2) (layer "F.Cu") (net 3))
 (segment (start 132.25 96.25) (end 135.25 99.25) (width 0.5) (layer "F.Cu") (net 3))
 (segment (start 135.25 103.75) (end 135.25 99.25) (width 0.5) (layer "F.Cu") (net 3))
 (segment (start 126.25 96.25) (end 132.25 96.25) (width 0.5) (layer "F.Cu") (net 3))
 (segment (start 131.5 130.5) (end 124.25 123.25) (width 0.2) (layer "F.Cu") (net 3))
 (via (at 135.25 102.25) (size 0.6) (drill 0.3) (layers "F.Cu" "B.Cu") (free yes) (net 3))
 (via (at 135.25 99.25) (size 0.6) (drill 0.3) (layers "F.Cu" "B.Cu") (free yes) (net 3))
 (via (at 126.25 94.75) (size 0.6) (drill 0.3) (layers "F.Cu" "B.Cu") (free yes) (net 3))
 (via (at 126.25 93.25) (size 0.6) (drill 0.3) (layers "F.Cu" "B.Cu") (free yes) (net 3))
 (via (at 126.25 91.75) (size 0.6) (drill 0.3) (layers "F.Cu" "B.Cu") (free yes) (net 3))
 (via (at 135.25 103.75) (size 0.6) (drill 0.3) (layers "F.Cu" "B.Cu") (free yes) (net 3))
 (via (at 126.25 96.25) (size 0.6) (drill 0.3) (layers "F.Cu" "B.Cu") (free yes) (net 3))
 (via (at 135.25 100.75) (size 0.6) (drill 0.3) (layers "F.Cu" "B.Cu") (free yes) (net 3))
 (segment (start 140.75 93.75) (end 135.25 99.25) (width 0.5) (layer "B.Cu") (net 3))
 (segment (start 127.55 88.4) (end 127.45 88.5) (width 0.2) (layer "B.Cu") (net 3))
 (segment (start 127.55 85.005) (end 127.55 88.4) (width 0.2) (layer "B.Cu") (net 3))
 (segment (start 127.55 85.005) (end 126.495 85.005) (width 0.5) (layer "B.Cu") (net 3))
 (segment (start 126.25 85.25) (end 126.25 96.25) (width 0.5) (layer "B.Cu") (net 3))
 (segment (start 126.495 85.005) (end 126.25 85.25) (width 0.5) (layer "B.Cu") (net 3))
 (segment (start 145.95 93.75) (end 140.75 93.75) (width 0.5) (layer "B.Cu") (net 3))
 (segment (start 117 111.25) (end 117 119) (width 0.5) (layer "B.Cu") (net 5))
 (segment (start 117.25 110.25) (end 117.25 111) (width 0.5) (layer "B.Cu") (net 5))
 (segment (start 145.95 85.75) (end 141.75 85.75) (width 0.5) (layer "B.Cu") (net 5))
 (segment (start 141.75 85.75) (end 117.25 110.25) (width 0.5) (layer "B.Cu") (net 5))
 (segment (start 117.25 111) (end 117 111.25) (width 0.5) (layer "B.Cu") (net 5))
 (segment (start 144.55237 115.83) (end 145.63 115.83) (width 0.2) (layer "F.Cu") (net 2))
 (segment (start 136.15 124.23237) (end 144.55237 115.83) (width 0.2) (layer "F.Cu") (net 2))
 (segment (start 136.15 128.75) (end 136.15 124.23237) (width 0.2) (layer "F.Cu") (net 2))
 (segment (start 132.75 125.09237) (end 132.75 128.75) (width 0.2) (layer "F.Cu") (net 1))
 (segment (start 144.55237 113.29) (end 132.75 125.09237) (width 0.2) (layer "F.Cu") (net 1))
 (segment (start 145.63 113.29) (end 144.55237 113.29) (width 0.2) (layer "F.Cu") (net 1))
 (segment (start 163.851 91.126) (end 163.851 107.769) (width 0.2) (layer "B.Cu") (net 15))
 (segment (start 161 89.75) (end 162.475 89.75) (width 0.2) (layer "B.Cu") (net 15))
 (segment (start 162.475 89.75) (end 163.851 91.126) (width 0.2) (layer "B.Cu") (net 15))
 (segment (start 163.851 107.769) (end 160.87 110.75) (width 0.2) (layer "B.Cu") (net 15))
 (segment (start 149.5 110.75) (end 158.75 101.5) (width 0.2) (layer "F.Cu") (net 10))
 (segment (start 158.75 101.5) (end 158.75 94.25) (width 0.2) (layer "F.Cu") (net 10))
 (segment (start 145.63 110.75) (end 149.5 110.75) (width 0.2) (layer "F.Cu") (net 10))
 (via (at 158.75 94.25) (size 0.6) (drill 0.3) (layers "F.Cu" "B.Cu") (free yes) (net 10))
 (segment (start 159.25 93.75) (end 161 93.75) (width 0.2) (layer "B.Cu") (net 10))
 (segment (start 158.75 94.25) (end 159.25 93.75) (width 0.2) (layer "B.Cu") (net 10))
 (segment (start 144.174 99.176308) (end 145.600308 97.75) (width 0.2) (layer "B.Cu") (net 8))
 (segment (start 145.63 105.67) (end 144.174 104.214) (width 0.2) (layer "B.Cu") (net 8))
 (segment (start 145.600308 97.75) (end 145.95 97.75) (width 0.2) (layer "B.Cu") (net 8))
 (segment (start 144.174 104.214) (end 144.174 99.176308) (width 0.2) (layer "B.Cu") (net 8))
 (segment (start 145.63 103.13) (end 145.63 100.07) (width 0.2) (layer "B.Cu") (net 7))
 (segment (start 145.63 100.07) (end 145.95 99.75) (width 0.2) (layer "B.Cu") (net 7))
 (segment (start 160.87 115.83) (end 158 112.96) (width 0.2) (layer "B.Cu") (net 13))
 (segment (start 158 112.96) (end 158 93.25) (width 0.2) (layer "B.Cu") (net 13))
 (segment (start 159.5 91.75) (end 161 91.75) (width 0.2) (layer "B.Cu") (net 13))
 (segment (start 158 93.25) (end 159.5 91.75) (width 0.2) (layer "B.Cu") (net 13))
 (segment (start 144.475 95.75) (end 145.95 95.75) (width 0.2) (layer "B.Cu") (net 9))
 (segment (start 145.63 108.21) (end 143 105.58) (width 0.2) (layer "B.Cu") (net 9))
 (segment (start 143 105.58) (end 143 97.225) (width 0.2) (layer "B.Cu") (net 9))
 (segment (start 143 97.225) (end 144.475 95.75) (width 0.2) (layer "B.Cu") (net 9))
 (segment (start 163.25 95.75) (end 164.25 95.75) (width 0.2) (layer "F.Cu") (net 12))
 (segment (start 165.5 97) (end 165.5 114.575) (width 0.2) (layer "F.Cu") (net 12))
 (segment (start 164.25 95.75) (end 165.5 97) (width 0.2) (layer "F.Cu") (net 12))
 (segment (start 165.5 114.575) (end 161.705 118.37) (width 0.2) (layer "F.Cu") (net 12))
 (via (at 163.25 95.75) (size 0.6) (drill 0.3) (layers "F.Cu" "B.Cu") (free yes) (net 12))
 (segment (start 163.25 95.75) (end 161 95.75) (width 0.2) (layer "B.Cu") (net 12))
 (segment (start 165.25 90.75) (end 162.25 87.75) (width 0.2) (layer "B.Cu") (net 14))
 (segment (start 165.25 108.91) (end 165.25 90.75) (width 0.2) (layer "B.Cu") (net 14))
 (segment (start 160.87 113.29) (end 165.25 108.91) (width 0.2) (layer "B.Cu") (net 14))
 (segment (start 162.25 87.75) (end 161 87.75) (width 0.2) (layer "B.Cu") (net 14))
 (segment (start 117.121 79.7911) (end 124.8461 79.7911) (width 0.2) (layer "B.Cu") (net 6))
 (segment (start 129.148999 81.589) (end 129.45 81.890001) (width 0.2) (layer "B.Cu") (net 6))
 (segment (start 128.162638 81.589) (end 129.148999 81.589) (width 0.2) (layer "B.Cu") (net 6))
 (segment (start 127.55 82.495) (end 127.55 82.201638) (width 0.2) (layer "B.Cu") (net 6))
 (segment (start 127.55 82.201638) (end 128.162638 81.589) (width 0.2) (layer "B.Cu") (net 6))
 (segment (start 129.45 81.890001) (end 129.45 82.495) (width 0.2) (layer "B.Cu") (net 6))
 (segment (start 124.8461 79.7911) (end 127.55 82.495) (width 0.2) (layer "B.Cu") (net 6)))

